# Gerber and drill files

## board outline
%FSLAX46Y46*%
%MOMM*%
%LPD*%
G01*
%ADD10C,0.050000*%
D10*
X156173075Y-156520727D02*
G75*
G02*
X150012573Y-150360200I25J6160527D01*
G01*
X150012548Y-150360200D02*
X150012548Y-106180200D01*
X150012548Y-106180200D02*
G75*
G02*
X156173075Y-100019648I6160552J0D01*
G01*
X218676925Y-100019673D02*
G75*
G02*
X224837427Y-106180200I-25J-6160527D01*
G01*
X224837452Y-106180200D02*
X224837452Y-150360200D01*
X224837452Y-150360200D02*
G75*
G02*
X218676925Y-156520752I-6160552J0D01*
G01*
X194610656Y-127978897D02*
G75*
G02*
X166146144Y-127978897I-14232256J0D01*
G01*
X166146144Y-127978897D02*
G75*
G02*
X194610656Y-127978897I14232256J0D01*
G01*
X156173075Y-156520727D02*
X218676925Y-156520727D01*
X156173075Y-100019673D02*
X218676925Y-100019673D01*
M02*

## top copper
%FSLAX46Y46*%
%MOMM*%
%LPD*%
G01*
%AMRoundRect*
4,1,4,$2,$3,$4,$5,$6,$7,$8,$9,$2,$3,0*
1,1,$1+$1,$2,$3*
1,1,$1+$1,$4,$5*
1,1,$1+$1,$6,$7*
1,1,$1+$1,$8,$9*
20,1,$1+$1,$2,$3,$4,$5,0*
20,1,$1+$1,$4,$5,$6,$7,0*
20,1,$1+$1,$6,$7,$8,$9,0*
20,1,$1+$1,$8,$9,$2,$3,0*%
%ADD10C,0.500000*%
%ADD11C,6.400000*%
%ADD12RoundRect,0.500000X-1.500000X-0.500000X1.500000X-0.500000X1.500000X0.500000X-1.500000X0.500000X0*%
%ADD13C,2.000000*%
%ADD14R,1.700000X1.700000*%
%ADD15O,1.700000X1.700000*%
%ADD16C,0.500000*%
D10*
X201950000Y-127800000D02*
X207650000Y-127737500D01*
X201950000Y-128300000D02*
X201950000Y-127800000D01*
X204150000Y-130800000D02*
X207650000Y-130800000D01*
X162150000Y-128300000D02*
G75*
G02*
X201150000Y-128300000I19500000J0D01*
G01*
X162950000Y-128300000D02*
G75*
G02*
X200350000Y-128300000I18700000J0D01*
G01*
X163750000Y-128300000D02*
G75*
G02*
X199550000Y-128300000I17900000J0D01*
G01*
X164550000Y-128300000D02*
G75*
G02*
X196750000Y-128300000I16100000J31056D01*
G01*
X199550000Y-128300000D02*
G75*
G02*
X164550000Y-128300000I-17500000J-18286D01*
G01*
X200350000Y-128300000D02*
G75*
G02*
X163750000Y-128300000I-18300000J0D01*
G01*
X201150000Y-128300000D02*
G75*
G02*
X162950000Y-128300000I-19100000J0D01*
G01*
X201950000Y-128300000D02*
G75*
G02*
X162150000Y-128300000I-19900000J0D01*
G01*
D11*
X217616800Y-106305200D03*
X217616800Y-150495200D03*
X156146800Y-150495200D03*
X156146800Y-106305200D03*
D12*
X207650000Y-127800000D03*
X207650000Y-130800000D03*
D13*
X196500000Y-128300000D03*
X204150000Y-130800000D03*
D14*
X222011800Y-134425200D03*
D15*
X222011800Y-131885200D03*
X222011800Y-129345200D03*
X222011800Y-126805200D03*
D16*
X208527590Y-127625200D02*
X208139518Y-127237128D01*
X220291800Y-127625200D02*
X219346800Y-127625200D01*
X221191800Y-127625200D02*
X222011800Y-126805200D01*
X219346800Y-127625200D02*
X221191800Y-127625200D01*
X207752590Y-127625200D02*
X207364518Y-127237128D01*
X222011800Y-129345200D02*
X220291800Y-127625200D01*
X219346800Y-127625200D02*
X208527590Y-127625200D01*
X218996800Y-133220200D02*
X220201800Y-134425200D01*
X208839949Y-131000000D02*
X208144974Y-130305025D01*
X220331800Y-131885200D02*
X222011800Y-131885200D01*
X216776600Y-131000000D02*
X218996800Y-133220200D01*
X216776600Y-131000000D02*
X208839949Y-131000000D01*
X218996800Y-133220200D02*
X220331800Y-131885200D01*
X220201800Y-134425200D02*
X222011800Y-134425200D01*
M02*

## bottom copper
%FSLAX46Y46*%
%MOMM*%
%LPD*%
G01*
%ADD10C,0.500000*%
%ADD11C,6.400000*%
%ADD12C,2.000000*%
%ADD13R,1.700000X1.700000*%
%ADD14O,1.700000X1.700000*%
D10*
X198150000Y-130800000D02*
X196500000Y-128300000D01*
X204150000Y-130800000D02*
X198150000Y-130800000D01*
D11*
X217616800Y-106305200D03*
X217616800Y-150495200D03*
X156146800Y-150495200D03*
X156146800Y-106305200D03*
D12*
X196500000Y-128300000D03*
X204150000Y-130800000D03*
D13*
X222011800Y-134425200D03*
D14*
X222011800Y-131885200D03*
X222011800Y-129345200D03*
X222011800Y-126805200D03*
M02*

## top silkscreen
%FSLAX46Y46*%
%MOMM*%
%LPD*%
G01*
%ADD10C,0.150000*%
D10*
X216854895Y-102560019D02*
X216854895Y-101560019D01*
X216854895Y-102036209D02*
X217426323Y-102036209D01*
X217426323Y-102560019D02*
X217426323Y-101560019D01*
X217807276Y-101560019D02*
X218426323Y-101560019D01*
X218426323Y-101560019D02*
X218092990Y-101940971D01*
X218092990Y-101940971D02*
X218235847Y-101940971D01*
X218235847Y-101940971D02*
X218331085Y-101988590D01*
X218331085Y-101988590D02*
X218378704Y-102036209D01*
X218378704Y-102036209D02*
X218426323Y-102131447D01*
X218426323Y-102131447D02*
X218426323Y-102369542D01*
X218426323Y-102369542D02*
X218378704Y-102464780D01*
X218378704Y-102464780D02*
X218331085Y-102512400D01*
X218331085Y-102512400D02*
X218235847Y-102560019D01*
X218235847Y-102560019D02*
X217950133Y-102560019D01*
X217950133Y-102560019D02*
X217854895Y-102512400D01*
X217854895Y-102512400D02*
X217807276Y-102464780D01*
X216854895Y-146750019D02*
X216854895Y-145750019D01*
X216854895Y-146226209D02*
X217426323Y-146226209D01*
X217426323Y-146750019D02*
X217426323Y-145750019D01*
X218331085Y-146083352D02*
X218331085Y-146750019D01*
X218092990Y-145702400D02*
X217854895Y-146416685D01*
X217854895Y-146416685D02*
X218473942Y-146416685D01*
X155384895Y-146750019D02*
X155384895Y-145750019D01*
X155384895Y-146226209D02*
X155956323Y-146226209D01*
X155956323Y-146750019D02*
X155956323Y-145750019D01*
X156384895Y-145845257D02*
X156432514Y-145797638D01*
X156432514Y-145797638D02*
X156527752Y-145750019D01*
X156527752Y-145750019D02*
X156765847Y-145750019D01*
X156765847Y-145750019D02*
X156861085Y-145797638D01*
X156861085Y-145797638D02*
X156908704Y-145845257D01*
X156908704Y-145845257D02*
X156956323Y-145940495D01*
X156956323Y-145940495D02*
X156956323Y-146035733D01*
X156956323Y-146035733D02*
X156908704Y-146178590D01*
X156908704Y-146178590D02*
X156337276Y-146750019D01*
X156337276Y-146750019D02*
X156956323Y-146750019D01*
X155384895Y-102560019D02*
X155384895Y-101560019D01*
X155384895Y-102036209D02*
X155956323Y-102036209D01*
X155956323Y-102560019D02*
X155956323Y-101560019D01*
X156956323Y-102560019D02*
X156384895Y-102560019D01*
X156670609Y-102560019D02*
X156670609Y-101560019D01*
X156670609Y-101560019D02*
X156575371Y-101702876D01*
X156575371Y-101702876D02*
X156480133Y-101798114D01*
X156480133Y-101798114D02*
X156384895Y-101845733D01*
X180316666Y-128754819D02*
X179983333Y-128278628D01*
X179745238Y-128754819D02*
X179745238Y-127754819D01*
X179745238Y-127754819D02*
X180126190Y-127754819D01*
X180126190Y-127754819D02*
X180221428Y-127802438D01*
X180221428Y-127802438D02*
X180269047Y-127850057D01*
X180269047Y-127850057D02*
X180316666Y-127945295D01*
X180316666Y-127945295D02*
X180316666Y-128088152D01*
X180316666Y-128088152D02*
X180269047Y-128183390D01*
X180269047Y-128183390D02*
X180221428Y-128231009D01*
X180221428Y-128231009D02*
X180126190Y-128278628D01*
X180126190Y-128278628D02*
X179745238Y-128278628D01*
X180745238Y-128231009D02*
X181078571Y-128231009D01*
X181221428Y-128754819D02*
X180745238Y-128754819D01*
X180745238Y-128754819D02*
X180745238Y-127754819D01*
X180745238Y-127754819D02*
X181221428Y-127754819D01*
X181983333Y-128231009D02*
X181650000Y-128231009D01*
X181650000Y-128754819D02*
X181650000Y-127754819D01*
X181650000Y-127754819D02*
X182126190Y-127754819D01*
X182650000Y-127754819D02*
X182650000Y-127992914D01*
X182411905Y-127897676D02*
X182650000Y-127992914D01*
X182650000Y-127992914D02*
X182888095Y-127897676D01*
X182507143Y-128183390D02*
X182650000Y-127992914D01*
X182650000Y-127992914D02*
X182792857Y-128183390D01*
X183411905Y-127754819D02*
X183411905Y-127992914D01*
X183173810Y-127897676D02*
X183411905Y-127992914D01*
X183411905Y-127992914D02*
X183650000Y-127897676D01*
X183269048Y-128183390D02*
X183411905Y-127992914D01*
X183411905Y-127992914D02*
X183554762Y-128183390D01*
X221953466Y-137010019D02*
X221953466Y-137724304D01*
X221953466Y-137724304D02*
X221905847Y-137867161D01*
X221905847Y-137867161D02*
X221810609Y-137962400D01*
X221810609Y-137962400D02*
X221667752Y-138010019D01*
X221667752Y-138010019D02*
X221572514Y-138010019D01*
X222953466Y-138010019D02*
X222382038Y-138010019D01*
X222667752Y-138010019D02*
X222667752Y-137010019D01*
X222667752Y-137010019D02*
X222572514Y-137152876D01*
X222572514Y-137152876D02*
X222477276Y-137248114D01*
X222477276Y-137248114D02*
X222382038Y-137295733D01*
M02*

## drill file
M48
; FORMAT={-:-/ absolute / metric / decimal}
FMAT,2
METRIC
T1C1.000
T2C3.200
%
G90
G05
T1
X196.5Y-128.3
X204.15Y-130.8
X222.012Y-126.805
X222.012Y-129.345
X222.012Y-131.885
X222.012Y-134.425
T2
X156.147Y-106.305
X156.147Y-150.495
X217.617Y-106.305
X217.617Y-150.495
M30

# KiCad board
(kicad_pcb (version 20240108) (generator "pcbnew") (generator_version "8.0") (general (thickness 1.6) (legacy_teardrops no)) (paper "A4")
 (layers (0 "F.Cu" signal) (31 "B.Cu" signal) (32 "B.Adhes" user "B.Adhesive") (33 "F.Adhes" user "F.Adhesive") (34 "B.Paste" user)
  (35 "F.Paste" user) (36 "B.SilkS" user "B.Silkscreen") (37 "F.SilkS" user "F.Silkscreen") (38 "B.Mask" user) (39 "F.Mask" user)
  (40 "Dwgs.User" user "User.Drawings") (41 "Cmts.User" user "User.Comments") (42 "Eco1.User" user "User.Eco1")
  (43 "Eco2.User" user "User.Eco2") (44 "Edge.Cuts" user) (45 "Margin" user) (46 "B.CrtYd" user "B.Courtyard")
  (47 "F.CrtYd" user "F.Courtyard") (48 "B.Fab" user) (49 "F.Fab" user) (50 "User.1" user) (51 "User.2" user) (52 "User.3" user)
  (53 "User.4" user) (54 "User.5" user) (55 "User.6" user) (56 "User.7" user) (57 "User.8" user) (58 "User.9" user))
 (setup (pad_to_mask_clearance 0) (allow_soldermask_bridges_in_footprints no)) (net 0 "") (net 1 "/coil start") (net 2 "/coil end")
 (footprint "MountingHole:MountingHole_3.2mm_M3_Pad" (layer "F.Cu") (at 217.6168 106.3052)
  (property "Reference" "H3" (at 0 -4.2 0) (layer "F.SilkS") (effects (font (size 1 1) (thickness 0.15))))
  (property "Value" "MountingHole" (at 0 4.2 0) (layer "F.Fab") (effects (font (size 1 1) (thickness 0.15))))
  (pad "1" thru_hole circle (at 0 0) (size 6.4 6.4) (drill 3.2) (layers "*.Cu" "*.Mask") (remove_unused_layers no)))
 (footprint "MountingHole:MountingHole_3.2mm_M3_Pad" (layer "F.Cu") (at 217.6168 150.4952)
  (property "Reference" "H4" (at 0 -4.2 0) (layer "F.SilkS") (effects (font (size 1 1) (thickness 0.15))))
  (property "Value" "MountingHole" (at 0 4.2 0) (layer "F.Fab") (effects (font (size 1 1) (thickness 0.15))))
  (pad "1" thru_hole circle (at 0 0) (size 6.4 6.4) (drill 3.2) (layers "*.Cu" "*.Mask") (remove_unused_layers no)))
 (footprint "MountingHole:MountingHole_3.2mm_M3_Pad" (layer "F.Cu") (at 156.1468 150.4952)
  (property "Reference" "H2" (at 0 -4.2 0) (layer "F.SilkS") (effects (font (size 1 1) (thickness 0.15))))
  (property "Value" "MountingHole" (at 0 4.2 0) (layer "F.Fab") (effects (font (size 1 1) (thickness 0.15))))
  (pad "1" thru_hole circle (at 0 0) (size 6.4 6.4) (drill 3.2) (layers "*.Cu" "*.Mask") (remove_unused_layers no)))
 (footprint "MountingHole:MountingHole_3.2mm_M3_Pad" (layer "F.Cu") (at 156.1468 106.3052)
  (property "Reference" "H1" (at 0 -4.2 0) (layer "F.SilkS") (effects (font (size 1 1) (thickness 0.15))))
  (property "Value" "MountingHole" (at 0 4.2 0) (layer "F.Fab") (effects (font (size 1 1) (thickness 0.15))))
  (pad "1" thru_hole circle (at 0 0) (size 6.4 6.4) (drill 3.2) (layers "*.Cu" "*.Mask") (remove_unused_layers no)))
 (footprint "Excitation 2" (layer "F.Cu") (at 181.65 128.3)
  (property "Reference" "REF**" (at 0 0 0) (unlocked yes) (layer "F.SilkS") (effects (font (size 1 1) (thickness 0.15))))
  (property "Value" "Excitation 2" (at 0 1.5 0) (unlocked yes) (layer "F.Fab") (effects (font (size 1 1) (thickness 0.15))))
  (fp_line (start 20.3 -0.5) (end 26 -0.5625) (stroke (width 0.5) (type solid)) (layer "F.Cu"))
  (fp_line (start 20.3 0) (end 20.3 -0.5) (stroke (width 0.5) (type solid)) (layer "F.Cu"))
  (fp_line (start 22.5 2.5) (end 26 2.5) (stroke (width 0.5) (type default)) (layer "F.Cu"))
  (fp_arc (start -19.5 0) (mid 0 -19.5) (end 19.5 0) (stroke (width 0.5) (type solid)) (layer "F.Cu"))
  (fp_arc (start -18.7 0) (mid 0 -18.7) (end 18.7 0) (stroke (width 0.5) (type solid)) (layer "F.Cu"))
  (fp_arc (start -17.9 0) (mid 0 -17.9) (end 17.9 0) (stroke (width 0.5) (type solid)) (layer "F.Cu"))
  (fp_arc (start -17.1 0) (mid -1 -16.131086) (end 15.1 0) (stroke (width 0.5) (type solid)) (layer "F.Cu"))
  (fp_arc (start 17.9 0) (mid 0.4 17.518296) (end -17.1 0) (stroke (width 0.5) (type solid)) (layer "F.Cu"))
  (fp_arc (start 18.7 0) (mid 0.4 18.3) (end -17.9 0) (stroke (width 0.5) (type solid)) (layer "F.Cu"))
  (fp_arc (start 19.5 0) (mid 0.4 19.1) (end -18.7 0) (stroke (width 0.5) (type solid)) (layer "F.Cu"))
  (fp_arc (start 20.3 0) (mid 0.4 19.9) (end -19.5 0) (stroke (width 0.5) (type solid)) (layer "F.Cu"))
  (fp_line (start 16.5 2.5) (end 14.85 0) (stroke (width 0.5) (type default)) (layer "B.Cu"))
  (fp_line (start 22.5 2.5) (end 16.5 2.5) (stroke (width 0.5) (type default)) (layer "B.Cu"))
  (pad "1" smd roundrect (at 26 -0.5) (size 4 2) (layers "F.Cu") (roundrect_rratio 0.25) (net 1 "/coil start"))
  (pad "2" smd roundrect (at 26 2.5) (size 4 2) (layers "F.Cu") (roundrect_rratio 0.25) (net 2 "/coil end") (thermal_bridge_angle 45))
  (pad "3" thru_hole circle (at 14.85 0) (size 2 2) (drill 1) (layers "*.Cu" "*.Mask") (remove_unused_layers no))
  (pad "3" thru_hole circle (at 22.5 2.5) (size 2 2) (drill 1) (layers "*.Cu" "*.Mask") (remove_unused_layers no)))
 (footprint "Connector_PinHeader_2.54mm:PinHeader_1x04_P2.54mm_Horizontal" (layer "B.Cu") (at 222.0118 134.4252)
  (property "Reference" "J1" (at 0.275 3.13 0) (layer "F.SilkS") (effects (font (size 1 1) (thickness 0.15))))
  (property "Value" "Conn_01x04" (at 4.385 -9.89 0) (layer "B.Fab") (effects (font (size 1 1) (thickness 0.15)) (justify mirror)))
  (pad "1" thru_hole rect (at 0 0) (size 1.7 1.7) (drill 1) (layers "*.Cu" "*.Mask") (remove_unused_layers no) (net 2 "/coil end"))
  (pad "2" thru_hole oval (at 0 -2.54) (size 1.7 1.7) (drill 1) (layers "*.Cu" "*.Mask") (remove_unused_layers no) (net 2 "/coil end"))
  (pad "3" thru_hole oval (at 0 -5.08) (size 1.7 1.7) (drill 1) (layers "*.Cu" "*.Mask") (remove_unused_layers no) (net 1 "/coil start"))
  (pad "4" thru_hole oval (at 0 -7.62) (size 1.7 1.7) (drill 1) (layers "*.Cu" "*.Mask") (remove_unused_layers no) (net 1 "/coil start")))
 (gr_arc (start 156.173075 156.520727) (mid 151.816925 154.71635) (end 150.012548 150.3602) (stroke (width 0.05) (type default))
  (layer "Edge.Cuts"))
 (gr_line (start 150.012548 150.3602) (end 150.012548 106.1802) (stroke (width 0.05) (type default)) (layer "Edge.Cuts"))
 (gr_arc (start 150.012548 106.1802) (mid 151.816925 101.82405) (end 156.173075 100.019673) (stroke (width 0.05) (type default))
  (layer "Edge.Cuts"))
 (gr_arc (start 218.676925 100.019673) (mid 223.033075 101.82405) (end 224.837452 106.1802) (stroke (width 0.05) (type default))
  (layer "Edge.Cuts"))
 (gr_line (start 224.837452 106.1802) (end 224.837452 150.3602) (stroke (width 0.05) (type default)) (layer "Edge.Cuts"))
 (gr_arc (start 224.837452 150.3602) (mid 223.033075 154.71635) (end 218.676925 156.520727) (stroke (width 0.05) (type default))
  (layer "Edge.Cuts"))
 (gr_circle (center 180.3784 127.978897) (end 192.7568 120.9552) (stroke (width 0.05) (type default)) (fill none) (layer "Edge.Cuts"))
 (gr_line (start 156.173075 156.520727) (end 218.676925 156.520727) (stroke (width 0.05) (type default)) (layer "Edge.Cuts"))
 (gr_line (start 156.173075 100.019673) (end 218.676925 100.019673) (stroke (width 0.05) (type default)) (layer "Edge.Cuts"))
 (segment (start 208.52759 127.6252) (end 208.139518 127.237128) (width 0.5) (layer "F.Cu") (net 1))
 (segment (start 220.2918 127.6252) (end 219.3468 127.6252) (width 0.5) (layer "F.Cu") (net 1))
 (segment (start 221.1918 127.6252) (end 222.0118 126.8052) (width 0.5) (layer "F.Cu") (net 1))
 (segment (start 219.3468 127.6252) (end 221.1918 127.6252) (width 0.5) (layer "F.Cu") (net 1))
 (segment (start 207.75259 127.6252) (end 207.364518 127.237128) (width 0.5) (layer "F.Cu") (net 1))
 (segment (start 222.0118 129.3452) (end 220.2918 127.6252) (width 0.5) (layer "F.Cu") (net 1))
 (segment (start 219.3468 127.6252) (end 208.52759 127.6252) (width 0.5) (layer "F.Cu") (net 1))
 (segment (start 218.9968 133.2202) (end 220.2018 134.4252) (width 0.5) (layer "F.Cu") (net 2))
 (segment (start 208.839949 131) (end 208.144974 130.305025) (width 0.5) (layer "F.Cu") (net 2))
 (segment (start 220.3318 131.8852) (end 222.0118 131.8852) (width 0.5) (layer "F.Cu") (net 2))
 (segment (start 216.7766 131) (end 218.9968 133.2202) (width 0.5) (layer "F.Cu") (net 2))
 (segment (start 216.7766 131) (end 208.839949 131) (width 0.5) (layer "F.Cu") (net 2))
 (segment (start 218.9968 133.2202) (end 220.3318 131.8852) (width 0.5) (layer "F.Cu") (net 2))
 (segment (start 220.2018 134.4252) (end 222.0118 134.4252) (width 0.5) (layer "F.Cu") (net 2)))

